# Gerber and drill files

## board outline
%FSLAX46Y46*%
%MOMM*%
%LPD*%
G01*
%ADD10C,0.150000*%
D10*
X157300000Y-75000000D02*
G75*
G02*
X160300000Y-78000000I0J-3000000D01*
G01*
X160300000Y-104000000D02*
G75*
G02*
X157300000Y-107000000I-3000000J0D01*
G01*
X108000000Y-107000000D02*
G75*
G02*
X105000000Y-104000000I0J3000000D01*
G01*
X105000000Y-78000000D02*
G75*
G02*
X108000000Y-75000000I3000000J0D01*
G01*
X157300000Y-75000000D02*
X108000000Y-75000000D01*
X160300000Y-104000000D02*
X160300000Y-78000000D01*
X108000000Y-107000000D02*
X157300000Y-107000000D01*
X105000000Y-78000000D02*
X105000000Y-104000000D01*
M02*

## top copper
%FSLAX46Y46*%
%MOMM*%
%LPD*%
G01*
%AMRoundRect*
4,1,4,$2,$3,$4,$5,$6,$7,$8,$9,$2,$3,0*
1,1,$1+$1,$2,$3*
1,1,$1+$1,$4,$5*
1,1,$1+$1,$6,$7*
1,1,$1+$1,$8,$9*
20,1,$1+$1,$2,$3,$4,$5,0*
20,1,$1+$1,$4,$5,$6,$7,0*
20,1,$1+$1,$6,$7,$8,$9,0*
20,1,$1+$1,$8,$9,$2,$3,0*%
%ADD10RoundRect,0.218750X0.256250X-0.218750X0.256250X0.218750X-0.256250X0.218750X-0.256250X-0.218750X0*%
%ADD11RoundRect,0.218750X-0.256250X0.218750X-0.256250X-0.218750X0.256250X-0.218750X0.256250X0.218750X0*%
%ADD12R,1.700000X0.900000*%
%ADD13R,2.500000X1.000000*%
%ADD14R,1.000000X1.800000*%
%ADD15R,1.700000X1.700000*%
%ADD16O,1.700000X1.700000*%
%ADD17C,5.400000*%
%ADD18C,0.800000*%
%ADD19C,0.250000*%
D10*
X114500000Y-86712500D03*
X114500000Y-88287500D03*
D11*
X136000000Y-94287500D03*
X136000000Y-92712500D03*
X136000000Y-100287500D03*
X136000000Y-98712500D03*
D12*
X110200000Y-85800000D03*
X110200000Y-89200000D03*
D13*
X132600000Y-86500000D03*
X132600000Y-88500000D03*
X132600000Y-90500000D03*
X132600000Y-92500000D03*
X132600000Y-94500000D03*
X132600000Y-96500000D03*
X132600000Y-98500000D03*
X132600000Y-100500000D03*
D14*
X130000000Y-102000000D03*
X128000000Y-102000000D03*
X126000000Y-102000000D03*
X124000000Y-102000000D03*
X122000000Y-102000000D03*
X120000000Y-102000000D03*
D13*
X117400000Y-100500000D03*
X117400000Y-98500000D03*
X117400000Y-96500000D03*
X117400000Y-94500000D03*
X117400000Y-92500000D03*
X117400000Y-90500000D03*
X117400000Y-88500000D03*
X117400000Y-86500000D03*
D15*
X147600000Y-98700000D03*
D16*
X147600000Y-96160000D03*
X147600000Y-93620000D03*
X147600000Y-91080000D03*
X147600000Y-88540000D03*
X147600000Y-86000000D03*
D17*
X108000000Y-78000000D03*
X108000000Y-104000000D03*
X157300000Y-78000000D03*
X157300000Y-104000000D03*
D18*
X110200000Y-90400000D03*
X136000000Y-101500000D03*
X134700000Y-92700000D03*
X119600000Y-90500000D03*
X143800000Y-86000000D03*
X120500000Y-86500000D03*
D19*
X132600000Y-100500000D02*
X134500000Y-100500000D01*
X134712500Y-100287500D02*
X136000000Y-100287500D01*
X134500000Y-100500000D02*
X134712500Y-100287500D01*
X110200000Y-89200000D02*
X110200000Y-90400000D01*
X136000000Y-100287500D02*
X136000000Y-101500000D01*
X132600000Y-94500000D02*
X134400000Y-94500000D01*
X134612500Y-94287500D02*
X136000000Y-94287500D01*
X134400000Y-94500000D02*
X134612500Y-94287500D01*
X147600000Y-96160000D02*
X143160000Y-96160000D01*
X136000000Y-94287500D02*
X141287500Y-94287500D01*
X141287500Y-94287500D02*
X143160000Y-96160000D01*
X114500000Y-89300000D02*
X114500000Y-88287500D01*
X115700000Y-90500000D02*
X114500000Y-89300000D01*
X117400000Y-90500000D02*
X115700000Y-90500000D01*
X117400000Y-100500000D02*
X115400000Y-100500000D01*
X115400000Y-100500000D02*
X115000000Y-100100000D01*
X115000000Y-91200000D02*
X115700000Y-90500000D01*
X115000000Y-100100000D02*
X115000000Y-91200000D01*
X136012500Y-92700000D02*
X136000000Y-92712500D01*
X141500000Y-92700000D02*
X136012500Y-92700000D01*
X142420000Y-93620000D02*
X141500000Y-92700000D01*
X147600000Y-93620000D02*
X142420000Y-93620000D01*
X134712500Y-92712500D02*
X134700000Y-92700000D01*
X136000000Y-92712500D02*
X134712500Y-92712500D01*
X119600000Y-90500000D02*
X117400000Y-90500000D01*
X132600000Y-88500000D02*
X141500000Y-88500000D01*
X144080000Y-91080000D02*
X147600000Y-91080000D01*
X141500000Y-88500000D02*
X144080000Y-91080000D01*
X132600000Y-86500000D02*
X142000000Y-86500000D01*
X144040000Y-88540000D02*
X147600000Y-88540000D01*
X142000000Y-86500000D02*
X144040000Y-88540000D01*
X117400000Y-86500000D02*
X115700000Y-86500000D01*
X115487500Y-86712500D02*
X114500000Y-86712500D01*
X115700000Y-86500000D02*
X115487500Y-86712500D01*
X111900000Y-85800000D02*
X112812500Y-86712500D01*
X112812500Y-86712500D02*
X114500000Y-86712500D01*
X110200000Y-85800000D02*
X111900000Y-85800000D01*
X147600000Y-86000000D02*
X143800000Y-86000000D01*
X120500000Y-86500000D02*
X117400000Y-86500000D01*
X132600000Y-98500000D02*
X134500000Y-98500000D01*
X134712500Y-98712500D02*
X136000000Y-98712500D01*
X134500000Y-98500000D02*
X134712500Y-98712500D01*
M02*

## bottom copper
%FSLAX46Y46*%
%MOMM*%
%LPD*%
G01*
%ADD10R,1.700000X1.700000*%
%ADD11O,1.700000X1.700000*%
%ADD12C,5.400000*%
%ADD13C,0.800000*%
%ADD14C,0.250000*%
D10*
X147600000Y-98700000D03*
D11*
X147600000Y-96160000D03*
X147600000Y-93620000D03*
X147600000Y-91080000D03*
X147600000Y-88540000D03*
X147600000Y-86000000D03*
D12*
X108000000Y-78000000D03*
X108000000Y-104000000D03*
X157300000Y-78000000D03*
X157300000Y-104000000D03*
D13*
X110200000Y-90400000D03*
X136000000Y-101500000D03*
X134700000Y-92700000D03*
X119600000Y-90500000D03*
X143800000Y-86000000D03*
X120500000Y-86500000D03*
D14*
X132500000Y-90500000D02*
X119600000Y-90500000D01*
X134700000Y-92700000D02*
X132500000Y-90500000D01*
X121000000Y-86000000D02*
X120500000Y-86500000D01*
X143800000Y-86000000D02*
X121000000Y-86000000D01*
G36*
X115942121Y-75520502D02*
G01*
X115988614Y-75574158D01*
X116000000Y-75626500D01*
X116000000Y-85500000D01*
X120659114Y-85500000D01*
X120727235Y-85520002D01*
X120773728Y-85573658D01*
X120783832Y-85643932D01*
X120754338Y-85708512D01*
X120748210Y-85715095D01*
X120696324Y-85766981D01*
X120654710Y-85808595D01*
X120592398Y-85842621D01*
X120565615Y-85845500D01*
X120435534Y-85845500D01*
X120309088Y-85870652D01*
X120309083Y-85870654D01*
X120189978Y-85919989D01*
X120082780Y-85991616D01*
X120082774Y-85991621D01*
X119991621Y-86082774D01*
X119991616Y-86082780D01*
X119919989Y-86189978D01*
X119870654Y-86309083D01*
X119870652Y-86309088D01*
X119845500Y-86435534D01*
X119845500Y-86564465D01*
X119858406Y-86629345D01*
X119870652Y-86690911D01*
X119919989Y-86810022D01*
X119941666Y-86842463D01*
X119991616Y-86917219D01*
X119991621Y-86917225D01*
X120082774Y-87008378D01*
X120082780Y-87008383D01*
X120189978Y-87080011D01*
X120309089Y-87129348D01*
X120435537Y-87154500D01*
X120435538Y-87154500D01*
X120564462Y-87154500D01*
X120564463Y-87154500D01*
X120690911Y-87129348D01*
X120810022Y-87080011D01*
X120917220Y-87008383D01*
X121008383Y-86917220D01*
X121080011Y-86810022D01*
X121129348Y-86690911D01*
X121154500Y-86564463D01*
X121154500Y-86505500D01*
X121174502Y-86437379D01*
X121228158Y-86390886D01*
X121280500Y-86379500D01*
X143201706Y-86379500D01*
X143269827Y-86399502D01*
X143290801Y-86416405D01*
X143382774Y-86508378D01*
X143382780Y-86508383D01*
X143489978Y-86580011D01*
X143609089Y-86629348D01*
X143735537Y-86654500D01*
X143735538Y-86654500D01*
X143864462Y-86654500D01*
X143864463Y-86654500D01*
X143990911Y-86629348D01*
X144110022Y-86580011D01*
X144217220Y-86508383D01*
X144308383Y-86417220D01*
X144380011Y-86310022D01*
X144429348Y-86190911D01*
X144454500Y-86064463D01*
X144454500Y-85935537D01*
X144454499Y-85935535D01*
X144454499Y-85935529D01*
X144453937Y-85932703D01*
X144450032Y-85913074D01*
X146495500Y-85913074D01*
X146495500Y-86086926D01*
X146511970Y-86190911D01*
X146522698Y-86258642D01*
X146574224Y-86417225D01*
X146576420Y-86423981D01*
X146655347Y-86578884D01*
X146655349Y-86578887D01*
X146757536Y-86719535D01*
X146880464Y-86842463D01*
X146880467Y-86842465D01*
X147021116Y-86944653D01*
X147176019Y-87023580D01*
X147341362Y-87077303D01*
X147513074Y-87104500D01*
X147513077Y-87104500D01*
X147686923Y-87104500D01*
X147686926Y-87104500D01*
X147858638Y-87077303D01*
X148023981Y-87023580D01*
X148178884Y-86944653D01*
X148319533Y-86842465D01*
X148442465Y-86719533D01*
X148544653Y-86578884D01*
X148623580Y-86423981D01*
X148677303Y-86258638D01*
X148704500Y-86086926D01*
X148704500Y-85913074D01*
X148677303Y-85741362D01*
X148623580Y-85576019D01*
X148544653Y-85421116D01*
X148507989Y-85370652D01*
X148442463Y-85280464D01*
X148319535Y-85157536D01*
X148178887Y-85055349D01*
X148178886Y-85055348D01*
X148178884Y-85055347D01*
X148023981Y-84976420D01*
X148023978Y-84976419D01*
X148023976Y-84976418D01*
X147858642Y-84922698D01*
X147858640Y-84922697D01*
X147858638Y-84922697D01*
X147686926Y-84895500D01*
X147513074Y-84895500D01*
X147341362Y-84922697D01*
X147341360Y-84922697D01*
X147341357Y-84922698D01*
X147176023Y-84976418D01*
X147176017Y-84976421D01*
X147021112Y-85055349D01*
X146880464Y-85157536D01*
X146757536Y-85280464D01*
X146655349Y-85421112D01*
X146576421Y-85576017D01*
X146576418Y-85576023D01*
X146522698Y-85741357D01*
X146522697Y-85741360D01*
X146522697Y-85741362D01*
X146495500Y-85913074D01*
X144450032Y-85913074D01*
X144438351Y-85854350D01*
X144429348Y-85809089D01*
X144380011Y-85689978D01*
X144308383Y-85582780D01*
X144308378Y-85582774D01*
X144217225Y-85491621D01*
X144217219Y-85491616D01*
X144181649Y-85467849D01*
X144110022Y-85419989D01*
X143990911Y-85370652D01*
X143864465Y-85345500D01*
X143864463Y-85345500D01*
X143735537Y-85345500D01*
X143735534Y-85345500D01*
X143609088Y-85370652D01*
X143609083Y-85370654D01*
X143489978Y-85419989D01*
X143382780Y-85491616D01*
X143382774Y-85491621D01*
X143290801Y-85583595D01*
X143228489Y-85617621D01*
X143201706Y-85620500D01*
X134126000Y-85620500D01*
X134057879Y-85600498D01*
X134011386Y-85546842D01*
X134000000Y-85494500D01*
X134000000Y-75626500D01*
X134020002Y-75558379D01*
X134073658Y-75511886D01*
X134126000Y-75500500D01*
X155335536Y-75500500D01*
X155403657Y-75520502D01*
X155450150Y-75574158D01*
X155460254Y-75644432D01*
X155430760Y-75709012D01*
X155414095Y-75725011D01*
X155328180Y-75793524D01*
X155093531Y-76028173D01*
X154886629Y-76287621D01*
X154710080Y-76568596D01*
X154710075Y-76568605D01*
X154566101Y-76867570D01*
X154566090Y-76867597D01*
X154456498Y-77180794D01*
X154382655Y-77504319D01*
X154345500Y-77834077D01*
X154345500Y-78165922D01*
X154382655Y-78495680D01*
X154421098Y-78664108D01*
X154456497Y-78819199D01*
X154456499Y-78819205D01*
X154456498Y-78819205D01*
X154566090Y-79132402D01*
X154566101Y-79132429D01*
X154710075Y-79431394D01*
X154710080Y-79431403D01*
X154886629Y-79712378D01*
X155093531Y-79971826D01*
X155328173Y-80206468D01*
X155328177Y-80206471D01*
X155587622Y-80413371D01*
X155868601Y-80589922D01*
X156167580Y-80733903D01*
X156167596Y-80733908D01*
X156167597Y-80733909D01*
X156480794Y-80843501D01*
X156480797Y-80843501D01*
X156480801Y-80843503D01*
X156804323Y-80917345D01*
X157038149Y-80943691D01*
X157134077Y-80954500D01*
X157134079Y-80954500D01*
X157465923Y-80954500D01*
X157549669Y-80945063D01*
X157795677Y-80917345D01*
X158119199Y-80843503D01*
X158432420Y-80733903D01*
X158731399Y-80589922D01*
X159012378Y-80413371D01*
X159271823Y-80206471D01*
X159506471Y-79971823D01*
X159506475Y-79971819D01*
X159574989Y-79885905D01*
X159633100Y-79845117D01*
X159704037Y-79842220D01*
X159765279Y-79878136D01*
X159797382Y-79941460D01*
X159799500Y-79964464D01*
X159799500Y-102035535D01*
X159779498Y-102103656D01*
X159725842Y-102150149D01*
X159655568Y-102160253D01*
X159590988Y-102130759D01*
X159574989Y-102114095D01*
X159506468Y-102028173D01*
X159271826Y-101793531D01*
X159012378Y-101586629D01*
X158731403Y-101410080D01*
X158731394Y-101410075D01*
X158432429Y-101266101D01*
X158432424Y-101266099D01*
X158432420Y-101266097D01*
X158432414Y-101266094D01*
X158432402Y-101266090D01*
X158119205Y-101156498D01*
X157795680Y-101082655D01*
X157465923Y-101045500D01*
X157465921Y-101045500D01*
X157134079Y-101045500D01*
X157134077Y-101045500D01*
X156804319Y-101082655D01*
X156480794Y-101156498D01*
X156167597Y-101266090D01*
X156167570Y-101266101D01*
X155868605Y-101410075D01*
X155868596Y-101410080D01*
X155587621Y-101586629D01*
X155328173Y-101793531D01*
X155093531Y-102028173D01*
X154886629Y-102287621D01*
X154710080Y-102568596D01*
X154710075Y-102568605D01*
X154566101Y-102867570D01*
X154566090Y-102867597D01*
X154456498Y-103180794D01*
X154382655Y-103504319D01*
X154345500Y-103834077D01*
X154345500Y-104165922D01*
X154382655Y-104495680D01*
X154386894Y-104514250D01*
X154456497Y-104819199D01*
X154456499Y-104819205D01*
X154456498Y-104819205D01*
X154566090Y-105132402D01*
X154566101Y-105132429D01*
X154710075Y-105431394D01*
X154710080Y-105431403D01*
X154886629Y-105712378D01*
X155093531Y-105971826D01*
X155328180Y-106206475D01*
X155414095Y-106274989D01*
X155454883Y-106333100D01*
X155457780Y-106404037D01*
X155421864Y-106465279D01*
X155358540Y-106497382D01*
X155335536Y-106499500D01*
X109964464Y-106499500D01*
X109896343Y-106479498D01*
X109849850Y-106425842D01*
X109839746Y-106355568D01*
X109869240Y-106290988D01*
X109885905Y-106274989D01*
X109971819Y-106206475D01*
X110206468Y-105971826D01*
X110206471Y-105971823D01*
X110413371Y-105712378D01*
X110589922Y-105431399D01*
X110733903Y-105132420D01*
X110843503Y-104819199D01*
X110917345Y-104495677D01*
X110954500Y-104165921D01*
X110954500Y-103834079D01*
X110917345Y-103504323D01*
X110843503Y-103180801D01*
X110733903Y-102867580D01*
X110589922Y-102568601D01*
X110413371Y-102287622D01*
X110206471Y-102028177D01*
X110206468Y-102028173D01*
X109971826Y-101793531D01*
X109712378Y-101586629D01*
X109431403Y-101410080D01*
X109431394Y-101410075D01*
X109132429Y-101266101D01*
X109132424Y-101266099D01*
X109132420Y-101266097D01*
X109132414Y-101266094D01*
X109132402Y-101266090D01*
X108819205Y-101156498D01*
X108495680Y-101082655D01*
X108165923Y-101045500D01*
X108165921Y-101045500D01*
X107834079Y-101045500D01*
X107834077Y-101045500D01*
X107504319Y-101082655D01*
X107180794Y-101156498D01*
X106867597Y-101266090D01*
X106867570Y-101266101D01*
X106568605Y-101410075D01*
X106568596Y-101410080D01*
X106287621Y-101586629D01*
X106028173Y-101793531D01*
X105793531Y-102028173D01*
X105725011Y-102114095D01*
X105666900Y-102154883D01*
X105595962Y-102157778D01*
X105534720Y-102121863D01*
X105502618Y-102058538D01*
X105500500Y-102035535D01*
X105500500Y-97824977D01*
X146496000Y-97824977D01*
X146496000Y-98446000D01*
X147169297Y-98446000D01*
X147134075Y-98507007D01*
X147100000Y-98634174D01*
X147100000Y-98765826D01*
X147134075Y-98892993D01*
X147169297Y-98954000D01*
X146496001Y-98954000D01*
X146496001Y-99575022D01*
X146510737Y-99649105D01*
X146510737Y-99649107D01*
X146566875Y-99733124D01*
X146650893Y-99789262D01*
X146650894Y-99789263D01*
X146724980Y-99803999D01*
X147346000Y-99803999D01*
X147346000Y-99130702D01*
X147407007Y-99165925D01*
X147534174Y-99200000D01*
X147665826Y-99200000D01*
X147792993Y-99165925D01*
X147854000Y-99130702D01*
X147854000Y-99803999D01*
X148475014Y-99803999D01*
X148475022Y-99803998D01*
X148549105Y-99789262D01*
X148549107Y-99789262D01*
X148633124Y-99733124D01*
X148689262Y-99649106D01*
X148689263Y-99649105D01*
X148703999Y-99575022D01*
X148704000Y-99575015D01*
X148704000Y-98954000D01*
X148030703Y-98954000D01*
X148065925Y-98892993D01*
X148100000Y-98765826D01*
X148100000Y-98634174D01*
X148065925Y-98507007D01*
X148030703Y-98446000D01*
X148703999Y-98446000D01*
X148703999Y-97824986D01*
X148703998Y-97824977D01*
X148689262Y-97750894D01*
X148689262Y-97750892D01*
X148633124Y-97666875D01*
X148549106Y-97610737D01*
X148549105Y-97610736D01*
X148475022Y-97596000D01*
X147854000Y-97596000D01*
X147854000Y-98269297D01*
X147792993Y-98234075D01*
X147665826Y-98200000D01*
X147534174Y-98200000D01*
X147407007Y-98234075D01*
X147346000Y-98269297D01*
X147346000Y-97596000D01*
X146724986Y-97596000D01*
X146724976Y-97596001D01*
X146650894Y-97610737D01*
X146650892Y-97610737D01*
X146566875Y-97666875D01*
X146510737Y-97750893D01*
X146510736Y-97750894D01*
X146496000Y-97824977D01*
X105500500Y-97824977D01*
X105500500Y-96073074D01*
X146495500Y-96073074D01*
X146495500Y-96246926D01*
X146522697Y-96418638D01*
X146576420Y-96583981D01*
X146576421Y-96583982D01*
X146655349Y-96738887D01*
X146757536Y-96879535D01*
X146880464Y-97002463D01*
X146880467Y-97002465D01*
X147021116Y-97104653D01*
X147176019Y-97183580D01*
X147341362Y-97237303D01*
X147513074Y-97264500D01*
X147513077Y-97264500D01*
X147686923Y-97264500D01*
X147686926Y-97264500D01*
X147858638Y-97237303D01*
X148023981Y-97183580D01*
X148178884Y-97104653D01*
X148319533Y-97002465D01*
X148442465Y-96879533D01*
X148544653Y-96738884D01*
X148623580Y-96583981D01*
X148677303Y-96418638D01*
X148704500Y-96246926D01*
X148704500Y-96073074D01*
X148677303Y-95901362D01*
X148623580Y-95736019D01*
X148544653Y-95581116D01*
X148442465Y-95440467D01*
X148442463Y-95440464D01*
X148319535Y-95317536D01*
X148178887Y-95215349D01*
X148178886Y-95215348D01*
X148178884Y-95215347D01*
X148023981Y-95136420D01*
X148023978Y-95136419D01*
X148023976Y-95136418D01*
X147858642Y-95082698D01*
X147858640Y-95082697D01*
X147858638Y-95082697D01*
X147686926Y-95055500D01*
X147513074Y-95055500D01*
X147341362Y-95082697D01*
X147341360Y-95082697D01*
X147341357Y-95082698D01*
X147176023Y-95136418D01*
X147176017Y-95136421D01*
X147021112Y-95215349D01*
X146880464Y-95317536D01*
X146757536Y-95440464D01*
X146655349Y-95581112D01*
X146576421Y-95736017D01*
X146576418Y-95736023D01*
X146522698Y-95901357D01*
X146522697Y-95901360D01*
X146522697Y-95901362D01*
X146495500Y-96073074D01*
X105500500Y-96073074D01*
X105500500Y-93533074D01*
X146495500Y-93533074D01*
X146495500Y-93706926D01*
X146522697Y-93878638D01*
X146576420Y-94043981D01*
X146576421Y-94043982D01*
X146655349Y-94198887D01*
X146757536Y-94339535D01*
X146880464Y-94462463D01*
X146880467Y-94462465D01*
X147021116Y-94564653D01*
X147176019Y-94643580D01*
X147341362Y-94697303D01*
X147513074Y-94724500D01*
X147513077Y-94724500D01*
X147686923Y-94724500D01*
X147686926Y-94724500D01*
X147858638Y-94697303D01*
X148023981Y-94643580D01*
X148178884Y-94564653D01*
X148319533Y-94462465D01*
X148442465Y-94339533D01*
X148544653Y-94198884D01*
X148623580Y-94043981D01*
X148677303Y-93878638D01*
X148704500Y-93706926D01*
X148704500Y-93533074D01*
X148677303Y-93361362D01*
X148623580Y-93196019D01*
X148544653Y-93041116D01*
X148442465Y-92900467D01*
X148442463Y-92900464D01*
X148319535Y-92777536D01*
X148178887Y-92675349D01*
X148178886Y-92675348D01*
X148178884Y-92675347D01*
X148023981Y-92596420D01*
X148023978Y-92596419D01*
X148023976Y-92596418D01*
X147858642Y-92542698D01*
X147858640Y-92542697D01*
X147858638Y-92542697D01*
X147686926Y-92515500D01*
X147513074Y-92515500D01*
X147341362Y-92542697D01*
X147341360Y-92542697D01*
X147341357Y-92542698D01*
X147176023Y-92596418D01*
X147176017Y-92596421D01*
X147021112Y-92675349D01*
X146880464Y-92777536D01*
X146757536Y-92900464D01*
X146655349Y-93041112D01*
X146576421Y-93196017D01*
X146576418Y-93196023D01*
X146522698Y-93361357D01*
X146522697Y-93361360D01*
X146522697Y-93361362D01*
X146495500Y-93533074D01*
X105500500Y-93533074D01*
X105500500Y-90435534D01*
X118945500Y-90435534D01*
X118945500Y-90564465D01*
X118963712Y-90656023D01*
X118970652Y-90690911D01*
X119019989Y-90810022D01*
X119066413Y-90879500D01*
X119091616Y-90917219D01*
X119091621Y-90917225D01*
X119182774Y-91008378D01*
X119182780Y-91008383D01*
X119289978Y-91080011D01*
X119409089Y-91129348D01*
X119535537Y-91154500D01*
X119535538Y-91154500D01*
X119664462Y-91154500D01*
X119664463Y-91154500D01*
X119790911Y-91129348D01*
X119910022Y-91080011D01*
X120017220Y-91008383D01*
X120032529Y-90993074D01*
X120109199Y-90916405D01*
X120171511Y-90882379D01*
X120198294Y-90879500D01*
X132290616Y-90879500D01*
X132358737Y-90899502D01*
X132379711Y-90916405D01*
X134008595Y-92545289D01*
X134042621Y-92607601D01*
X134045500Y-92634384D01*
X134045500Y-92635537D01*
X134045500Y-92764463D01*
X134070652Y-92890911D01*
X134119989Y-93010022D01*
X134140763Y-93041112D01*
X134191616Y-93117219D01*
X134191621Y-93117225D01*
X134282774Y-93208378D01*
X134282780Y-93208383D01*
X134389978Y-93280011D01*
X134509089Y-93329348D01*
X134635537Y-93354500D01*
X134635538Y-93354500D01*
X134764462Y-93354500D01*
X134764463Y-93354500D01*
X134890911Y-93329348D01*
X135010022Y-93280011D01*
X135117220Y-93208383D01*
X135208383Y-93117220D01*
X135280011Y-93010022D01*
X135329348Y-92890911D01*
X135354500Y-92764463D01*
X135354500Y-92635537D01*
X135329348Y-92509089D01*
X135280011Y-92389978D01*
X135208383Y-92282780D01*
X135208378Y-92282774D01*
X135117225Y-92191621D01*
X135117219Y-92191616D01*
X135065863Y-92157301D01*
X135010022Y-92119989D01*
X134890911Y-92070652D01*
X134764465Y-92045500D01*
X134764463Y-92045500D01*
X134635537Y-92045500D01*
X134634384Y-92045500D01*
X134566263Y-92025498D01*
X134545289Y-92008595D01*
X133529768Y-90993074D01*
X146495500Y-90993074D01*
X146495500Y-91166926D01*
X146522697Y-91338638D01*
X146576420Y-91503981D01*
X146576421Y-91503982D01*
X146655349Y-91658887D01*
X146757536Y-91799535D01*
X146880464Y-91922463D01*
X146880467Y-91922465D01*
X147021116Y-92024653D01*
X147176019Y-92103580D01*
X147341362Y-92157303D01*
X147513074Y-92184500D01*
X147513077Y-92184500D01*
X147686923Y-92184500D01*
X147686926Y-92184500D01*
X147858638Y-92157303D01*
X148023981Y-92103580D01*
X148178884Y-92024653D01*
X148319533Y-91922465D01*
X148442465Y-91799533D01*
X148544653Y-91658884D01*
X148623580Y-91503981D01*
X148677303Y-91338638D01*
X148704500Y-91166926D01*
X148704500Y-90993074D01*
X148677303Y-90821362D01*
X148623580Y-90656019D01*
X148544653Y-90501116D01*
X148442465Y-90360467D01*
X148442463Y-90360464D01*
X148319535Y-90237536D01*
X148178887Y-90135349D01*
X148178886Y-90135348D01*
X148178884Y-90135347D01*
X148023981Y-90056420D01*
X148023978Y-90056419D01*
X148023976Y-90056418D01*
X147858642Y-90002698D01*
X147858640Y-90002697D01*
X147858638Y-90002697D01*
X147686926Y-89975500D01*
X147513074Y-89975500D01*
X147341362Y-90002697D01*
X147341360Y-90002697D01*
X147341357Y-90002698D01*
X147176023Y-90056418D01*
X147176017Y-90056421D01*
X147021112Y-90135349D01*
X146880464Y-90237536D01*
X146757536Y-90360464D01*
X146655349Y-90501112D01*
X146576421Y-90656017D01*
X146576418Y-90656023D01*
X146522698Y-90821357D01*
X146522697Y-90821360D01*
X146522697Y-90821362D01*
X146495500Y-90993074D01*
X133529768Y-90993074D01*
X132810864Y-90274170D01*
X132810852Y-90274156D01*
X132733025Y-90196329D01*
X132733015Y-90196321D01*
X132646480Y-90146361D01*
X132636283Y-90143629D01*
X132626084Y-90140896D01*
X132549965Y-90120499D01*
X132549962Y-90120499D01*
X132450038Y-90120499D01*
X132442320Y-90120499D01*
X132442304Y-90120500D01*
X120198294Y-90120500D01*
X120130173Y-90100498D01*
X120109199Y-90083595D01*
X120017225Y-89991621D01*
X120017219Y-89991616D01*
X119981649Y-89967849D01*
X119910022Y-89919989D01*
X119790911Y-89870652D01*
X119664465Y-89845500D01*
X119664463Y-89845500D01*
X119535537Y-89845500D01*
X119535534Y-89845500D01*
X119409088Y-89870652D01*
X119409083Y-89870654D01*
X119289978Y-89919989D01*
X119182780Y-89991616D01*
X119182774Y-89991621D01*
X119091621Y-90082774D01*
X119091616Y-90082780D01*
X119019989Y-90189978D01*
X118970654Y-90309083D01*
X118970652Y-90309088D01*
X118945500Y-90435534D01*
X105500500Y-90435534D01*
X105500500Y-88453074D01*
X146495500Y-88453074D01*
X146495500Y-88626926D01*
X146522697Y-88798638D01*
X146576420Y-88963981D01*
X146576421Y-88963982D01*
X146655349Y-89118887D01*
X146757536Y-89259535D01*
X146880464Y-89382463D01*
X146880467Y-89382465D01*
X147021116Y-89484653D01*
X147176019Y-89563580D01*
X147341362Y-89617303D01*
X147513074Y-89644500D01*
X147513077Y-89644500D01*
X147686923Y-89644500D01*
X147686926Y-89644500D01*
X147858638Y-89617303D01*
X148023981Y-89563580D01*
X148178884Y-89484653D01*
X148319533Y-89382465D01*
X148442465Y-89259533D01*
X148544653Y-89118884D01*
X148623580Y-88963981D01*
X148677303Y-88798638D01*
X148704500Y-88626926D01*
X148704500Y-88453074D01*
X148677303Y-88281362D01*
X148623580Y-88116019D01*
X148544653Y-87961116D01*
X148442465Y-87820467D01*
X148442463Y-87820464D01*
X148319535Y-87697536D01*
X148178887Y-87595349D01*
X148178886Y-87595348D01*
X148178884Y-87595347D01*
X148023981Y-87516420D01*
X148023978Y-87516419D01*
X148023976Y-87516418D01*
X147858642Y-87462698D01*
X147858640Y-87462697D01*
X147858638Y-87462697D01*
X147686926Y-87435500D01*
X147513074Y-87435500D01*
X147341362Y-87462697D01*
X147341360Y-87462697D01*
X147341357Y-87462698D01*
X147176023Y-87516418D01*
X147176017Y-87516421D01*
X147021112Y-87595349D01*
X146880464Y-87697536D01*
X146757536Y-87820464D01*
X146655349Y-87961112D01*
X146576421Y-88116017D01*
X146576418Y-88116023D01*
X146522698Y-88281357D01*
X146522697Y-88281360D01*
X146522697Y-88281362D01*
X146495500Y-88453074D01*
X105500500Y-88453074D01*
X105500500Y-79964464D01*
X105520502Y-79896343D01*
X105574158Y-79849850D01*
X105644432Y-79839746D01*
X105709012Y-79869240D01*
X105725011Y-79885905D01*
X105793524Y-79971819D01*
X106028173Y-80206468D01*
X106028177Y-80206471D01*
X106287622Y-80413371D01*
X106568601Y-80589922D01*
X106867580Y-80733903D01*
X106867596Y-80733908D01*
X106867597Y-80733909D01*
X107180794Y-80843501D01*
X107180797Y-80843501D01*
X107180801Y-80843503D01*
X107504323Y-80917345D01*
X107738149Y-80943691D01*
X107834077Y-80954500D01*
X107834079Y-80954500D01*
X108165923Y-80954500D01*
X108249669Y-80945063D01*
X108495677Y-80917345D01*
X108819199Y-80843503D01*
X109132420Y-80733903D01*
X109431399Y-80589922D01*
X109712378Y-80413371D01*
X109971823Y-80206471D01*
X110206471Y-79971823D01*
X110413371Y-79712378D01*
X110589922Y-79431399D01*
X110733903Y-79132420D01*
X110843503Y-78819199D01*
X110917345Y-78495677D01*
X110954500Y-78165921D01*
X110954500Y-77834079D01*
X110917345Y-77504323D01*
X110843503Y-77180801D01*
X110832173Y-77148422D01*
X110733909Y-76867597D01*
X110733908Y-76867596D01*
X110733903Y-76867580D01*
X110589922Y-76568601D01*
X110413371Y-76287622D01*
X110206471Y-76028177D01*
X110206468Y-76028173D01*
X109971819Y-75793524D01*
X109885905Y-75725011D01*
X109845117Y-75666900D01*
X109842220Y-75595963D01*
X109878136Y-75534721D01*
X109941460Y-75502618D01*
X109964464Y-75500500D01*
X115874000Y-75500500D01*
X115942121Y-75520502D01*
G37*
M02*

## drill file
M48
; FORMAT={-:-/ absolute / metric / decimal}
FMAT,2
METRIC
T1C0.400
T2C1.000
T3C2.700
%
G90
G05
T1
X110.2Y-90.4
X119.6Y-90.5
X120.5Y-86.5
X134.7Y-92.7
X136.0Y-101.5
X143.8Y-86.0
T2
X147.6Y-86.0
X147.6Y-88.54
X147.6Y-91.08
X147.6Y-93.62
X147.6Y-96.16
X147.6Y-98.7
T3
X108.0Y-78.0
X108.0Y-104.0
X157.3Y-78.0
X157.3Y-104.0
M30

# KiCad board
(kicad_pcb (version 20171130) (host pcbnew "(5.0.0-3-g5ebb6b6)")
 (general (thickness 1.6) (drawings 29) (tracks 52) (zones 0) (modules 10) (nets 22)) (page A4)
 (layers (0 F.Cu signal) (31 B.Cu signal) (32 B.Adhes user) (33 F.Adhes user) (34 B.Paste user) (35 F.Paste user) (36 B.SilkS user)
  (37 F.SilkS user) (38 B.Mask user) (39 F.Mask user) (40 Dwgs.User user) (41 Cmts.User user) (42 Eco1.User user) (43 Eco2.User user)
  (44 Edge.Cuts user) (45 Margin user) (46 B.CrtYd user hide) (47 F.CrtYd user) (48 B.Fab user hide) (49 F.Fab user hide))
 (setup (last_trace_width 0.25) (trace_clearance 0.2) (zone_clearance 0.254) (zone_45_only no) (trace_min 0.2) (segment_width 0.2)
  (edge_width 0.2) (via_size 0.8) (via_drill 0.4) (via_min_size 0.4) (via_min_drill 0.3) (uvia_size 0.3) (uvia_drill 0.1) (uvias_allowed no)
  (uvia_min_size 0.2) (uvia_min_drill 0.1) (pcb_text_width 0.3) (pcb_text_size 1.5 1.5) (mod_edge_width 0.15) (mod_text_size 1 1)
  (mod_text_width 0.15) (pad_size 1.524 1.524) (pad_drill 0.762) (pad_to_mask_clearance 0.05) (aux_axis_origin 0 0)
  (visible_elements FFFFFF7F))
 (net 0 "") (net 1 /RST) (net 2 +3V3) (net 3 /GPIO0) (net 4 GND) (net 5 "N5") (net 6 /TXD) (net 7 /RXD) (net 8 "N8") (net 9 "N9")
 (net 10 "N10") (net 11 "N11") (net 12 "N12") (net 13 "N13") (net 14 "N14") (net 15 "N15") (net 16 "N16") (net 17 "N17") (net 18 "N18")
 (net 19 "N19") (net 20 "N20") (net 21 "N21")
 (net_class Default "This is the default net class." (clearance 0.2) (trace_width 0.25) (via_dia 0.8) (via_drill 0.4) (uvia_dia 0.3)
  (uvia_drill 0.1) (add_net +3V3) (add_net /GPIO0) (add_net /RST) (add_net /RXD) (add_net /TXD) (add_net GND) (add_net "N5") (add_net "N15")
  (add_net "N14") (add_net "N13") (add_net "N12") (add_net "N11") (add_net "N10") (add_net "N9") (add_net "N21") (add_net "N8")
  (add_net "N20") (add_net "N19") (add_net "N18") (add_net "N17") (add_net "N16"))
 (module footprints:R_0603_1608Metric (layer F.Cu) (at 114.5 87.5 90)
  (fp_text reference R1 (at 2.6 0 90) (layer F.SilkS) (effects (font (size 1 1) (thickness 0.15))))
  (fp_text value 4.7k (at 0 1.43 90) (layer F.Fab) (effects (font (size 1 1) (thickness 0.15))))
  (pad 2 smd roundrect (at 0.7875 0 90) (size 0.875 0.95) (layers F.Cu F.Paste F.Mask) (roundrect_rratio 0.25) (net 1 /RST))
  (pad 1 smd roundrect (at -0.7875 0 90) (size 0.875 0.95) (layers F.Cu F.Paste F.Mask) (roundrect_rratio 0.25) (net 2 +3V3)))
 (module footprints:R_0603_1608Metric (layer F.Cu) (at 136 93.5 270)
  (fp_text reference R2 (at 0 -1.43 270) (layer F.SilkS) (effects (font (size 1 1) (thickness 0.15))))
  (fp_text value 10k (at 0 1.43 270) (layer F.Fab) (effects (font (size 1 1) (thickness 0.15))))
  (pad 2 smd roundrect (at 0.7875 0 270) (size 0.875 0.95) (layers F.Cu F.Paste F.Mask) (roundrect_rratio 0.25) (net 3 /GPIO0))
  (pad 1 smd roundrect (at -0.7875 0 270) (size 0.875 0.95) (layers F.Cu F.Paste F.Mask) (roundrect_rratio 0.25) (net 2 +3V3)))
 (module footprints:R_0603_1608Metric (layer F.Cu) (at 136 99.5 270)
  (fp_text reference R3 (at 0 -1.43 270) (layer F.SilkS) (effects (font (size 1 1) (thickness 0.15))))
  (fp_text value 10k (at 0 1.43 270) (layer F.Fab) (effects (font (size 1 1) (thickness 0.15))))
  (pad 2 smd roundrect (at 0.7875 0 270) (size 0.875 0.95) (layers F.Cu F.Paste F.Mask) (roundrect_rratio 0.25) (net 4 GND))
  (pad 1 smd roundrect (at -0.7875 0 270) (size 0.875 0.95) (layers F.Cu F.Paste F.Mask) (roundrect_rratio 0.25) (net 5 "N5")))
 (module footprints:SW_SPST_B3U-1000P (layer F.Cu) (at 110.2 87.5 90)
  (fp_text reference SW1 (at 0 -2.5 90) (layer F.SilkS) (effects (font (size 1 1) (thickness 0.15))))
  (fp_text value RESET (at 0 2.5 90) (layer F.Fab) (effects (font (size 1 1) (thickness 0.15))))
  (pad 2 smd rect (at 1.7 0 90) (size 0.9 1.7) (layers F.Cu F.Paste F.Mask) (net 1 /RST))
  (pad 1 smd rect (at -1.7 0 90) (size 0.9 1.7) (layers F.Cu F.Paste F.Mask) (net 4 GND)))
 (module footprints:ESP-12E (layer F.Cu) (at 125 90)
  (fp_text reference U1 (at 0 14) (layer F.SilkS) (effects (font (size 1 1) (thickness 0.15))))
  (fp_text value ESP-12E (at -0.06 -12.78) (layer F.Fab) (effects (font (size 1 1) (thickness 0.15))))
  (pad 22 smd rect (at 7.6 -3.5) (size 2.5 1) (layers F.Cu F.Paste F.Mask) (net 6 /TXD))
  (pad 21 smd rect (at 7.6 -1.5) (size 2.5 1) (layers F.Cu F.Paste F.Mask) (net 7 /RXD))
  (pad 20 smd rect (at 7.6 0.5) (size 2.5 1) (layers F.Cu F.Paste F.Mask) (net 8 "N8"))
  (pad 19 smd rect (at 7.6 2.5) (size 2.5 1) (layers F.Cu F.Paste F.Mask) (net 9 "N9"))
  (pad 18 smd rect (at 7.6 4.5) (size 2.5 1) (layers F.Cu F.Paste F.Mask) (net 3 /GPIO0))
  (pad 17 smd rect (at 7.6 6.5) (size 2.5 1) (layers F.Cu F.Paste F.Mask) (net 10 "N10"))
  (pad 16 smd rect (at 7.6 8.5) (size 2.5 1) (layers F.Cu F.Paste F.Mask) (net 5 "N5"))
  (pad 15 smd rect (at 7.6 10.5) (size 2.5 1) (layers F.Cu F.Paste F.Mask) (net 4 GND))
  (pad 14 smd rect (at 5 12) (size 1 1.8) (layers F.Cu F.Paste F.Mask) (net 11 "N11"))
  (pad 13 smd rect (at 3 12) (size 1 1.8) (layers F.Cu F.Paste F.Mask) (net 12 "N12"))
  (pad 12 smd rect (at 1 12) (size 1 1.8) (layers F.Cu F.Paste F.Mask) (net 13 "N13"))
  (pad 11 smd rect (at -1 12) (size 1 1.8) (layers F.Cu F.Paste F.Mask) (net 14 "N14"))
  (pad 10 smd rect (at -3 12) (size 1 1.8) (layers F.Cu F.Paste F.Mask) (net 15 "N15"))
  (pad 9 smd rect (at -5 12) (size 1 1.8) (layers F.Cu F.Paste F.Mask) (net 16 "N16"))
  (pad 8 smd rect (at -7.6 10.5) (size 2.5 1) (layers F.Cu F.Paste F.Mask) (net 2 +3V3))
  (pad 7 smd rect (at -7.6 8.5) (size 2.5 1) (layers F.Cu F.Paste F.Mask) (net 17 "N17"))
  (pad 6 smd rect (at -7.6 6.5) (size 2.5 1) (layers F.Cu F.Paste F.Mask) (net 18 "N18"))
  (pad 5 smd rect (at -7.6 4.5) (size 2.5 1) (layers F.Cu F.Paste F.Mask) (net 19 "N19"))
  (pad 4 smd rect (at -7.6 2.5) (size 2.5 1) (layers F.Cu F.Paste F.Mask) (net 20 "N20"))
  (pad 3 smd rect (at -7.6 0.5) (size 2.5 1) (layers F.Cu F.Paste F.Mask) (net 2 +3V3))
  (pad 2 smd rect (at -7.6 -1.5) (size 2.5 1) (layers F.Cu F.Paste F.Mask) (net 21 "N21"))
  (pad 1 smd rect (at -7.6 -3.5) (size 2.5 1) (layers F.Cu F.Paste F.Mask) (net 1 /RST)))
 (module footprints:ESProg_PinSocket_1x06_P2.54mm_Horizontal (layer F.Cu) (at 147.6 98.7)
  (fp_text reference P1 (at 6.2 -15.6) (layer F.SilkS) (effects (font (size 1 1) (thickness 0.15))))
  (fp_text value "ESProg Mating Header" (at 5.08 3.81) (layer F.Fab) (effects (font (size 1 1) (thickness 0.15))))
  (pad 1 thru_hole rect (at 0 0 180) (size 1.7 1.7) (drill 1) (layers *.Cu *.Mask) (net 4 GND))
  (pad 2 thru_hole oval (at 0 -2.54 180) (size 1.7 1.7) (drill 1) (layers *.Cu *.Mask) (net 3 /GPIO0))
  (pad 3 thru_hole oval (at 0 -5.08 180) (size 1.7 1.7) (drill 1) (layers *.Cu *.Mask) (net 2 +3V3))
  (pad 4 thru_hole oval (at 0 -7.62 180) (size 1.7 1.7) (drill 1) (layers *.Cu *.Mask) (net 7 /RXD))
  (pad 5 thru_hole oval (at 0 -10.16 180) (size 1.7 1.7) (drill 1) (layers *.Cu *.Mask) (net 6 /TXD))
  (pad 6 thru_hole oval (at 0 -12.7 180) (size 1.7 1.7) (drill 1) (layers *.Cu *.Mask) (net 1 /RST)))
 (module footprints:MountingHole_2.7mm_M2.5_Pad (layer F.Cu) (at 108 78)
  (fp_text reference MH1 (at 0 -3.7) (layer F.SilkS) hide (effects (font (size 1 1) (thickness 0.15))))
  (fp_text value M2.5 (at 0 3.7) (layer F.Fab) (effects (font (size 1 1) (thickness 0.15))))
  (pad 1 thru_hole circle (at 0 0) (size 5.4 5.4) (drill 2.7) (layers *.Cu *.Mask)))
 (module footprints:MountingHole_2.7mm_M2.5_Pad (layer F.Cu) (at 108 104)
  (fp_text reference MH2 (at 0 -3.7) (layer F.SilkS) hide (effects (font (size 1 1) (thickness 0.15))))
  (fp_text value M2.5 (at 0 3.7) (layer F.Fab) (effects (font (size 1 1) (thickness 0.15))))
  (pad 1 thru_hole circle (at 0 0) (size 5.4 5.4) (drill 2.7) (layers *.Cu *.Mask)))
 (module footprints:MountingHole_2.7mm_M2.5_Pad (layer F.Cu) (at 157.3 78)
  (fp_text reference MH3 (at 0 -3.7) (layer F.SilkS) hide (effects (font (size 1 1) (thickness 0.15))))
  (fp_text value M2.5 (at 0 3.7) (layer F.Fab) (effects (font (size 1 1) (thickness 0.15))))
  (pad 1 thru_hole circle (at 0 0) (size 5.4 5.4) (drill 2.7) (layers *.Cu *.Mask)))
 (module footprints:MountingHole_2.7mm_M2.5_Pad (layer F.Cu) (at 157.3 104)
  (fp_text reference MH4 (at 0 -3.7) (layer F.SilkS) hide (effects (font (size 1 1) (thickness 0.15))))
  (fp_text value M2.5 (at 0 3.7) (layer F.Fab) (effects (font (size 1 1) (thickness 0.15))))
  (pad 1 thru_hole circle (at 0 0) (size 5.4 5.4) (drill 2.7) (layers *.Cu *.Mask)))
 (gr_arc (start 157.3 78) (end 160.3 78) (angle -90) (layer Edge.Cuts) (width 0.15))
 (gr_arc (start 157.3 104) (end 157.3 107) (angle -90) (layer Edge.Cuts) (width 0.15))
 (gr_arc (start 108 104) (end 105 104) (angle -90) (layer Edge.Cuts) (width 0.15))
 (gr_arc (start 108 78) (end 108 75) (angle -90) (layer Edge.Cuts) (width 0.15))
 (gr_line (start 157.3 75) (end 108 75) (layer Edge.Cuts) (width 0.15))
 (gr_line (start 160.3 104) (end 160.3 78) (layer Edge.Cuts) (width 0.15))
 (gr_line (start 108 107) (end 157.3 107) (layer Edge.Cuts) (width 0.15))
 (gr_line (start 105 78) (end 105 104) (layer Edge.Cuts) (width 0.15))
 (segment (start 132.6 100.5) (end 134.5 100.5) (width 0.25) (layer F.Cu) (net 4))
 (segment (start 134.7125 100.2875) (end 136 100.2875) (width 0.25) (layer F.Cu) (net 4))
 (segment (start 134.5 100.5) (end 134.7125 100.2875) (width 0.25) (layer F.Cu) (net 4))
 (via (at 110.2 90.4) (size 0.8) (drill 0.4) (layers F.Cu B.Cu) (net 4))
 (segment (start 110.2 89.2) (end 110.2 90.4) (width 0.25) (layer F.Cu) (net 4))
 (via (at 136 101.5) (size 0.8) (drill 0.4) (layers F.Cu B.Cu) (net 4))
 (segment (start 136 100.2875) (end 136 101.5) (width 0.25) (layer F.Cu) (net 4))
 (segment (start 132.6 94.5) (end 134.4 94.5) (width 0.25) (layer F.Cu) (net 3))
 (segment (start 134.6125 94.2875) (end 136 94.2875) (width 0.25) (layer F.Cu) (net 3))
 (segment (start 134.4 94.5) (end 134.6125 94.2875) (width 0.25) (layer F.Cu) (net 3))
 (segment (start 147.6 96.16) (end 143.16 96.16) (width 0.25) (layer F.Cu) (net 3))
 (segment (start 136 94.2875) (end 141.2875 94.2875) (width 0.25) (layer F.Cu) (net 3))
 (segment (start 141.2875 94.2875) (end 143.16 96.16) (width 0.25) (layer F.Cu) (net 3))
 (segment (start 114.5 89.3) (end 114.5 88.2875) (width 0.25) (layer F.Cu) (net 2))
 (segment (start 115.7 90.5) (end 114.5 89.3) (width 0.25) (layer F.Cu) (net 2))
 (segment (start 117.4 90.5) (end 115.7 90.5) (width 0.25) (layer F.Cu) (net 2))
 (segment (start 117.4 100.5) (end 115.4 100.5) (width 0.25) (layer F.Cu) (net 2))
 (segment (start 115.4 100.5) (end 115 100.1) (width 0.25) (layer F.Cu) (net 2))
 (segment (start 115 91.2) (end 115.7 90.5) (width 0.25) (layer F.Cu) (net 2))
 (segment (start 115 100.1) (end 115 91.2) (width 0.25) (layer F.Cu) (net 2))
 (segment (start 136.0125 92.7) (end 136 92.7125) (width 0.25) (layer F.Cu) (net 2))
 (segment (start 141.5 92.7) (end 136.0125 92.7) (width 0.25) (layer F.Cu) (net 2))
 (segment (start 142.42 93.62) (end 141.5 92.7) (width 0.25) (layer F.Cu) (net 2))
 (segment (start 147.6 93.62) (end 142.42 93.62) (width 0.25) (layer F.Cu) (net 2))
 (via (at 134.7 92.7) (size 0.8) (drill 0.4) (layers F.Cu B.Cu) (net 2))
 (segment (start 134.7125 92.7125) (end 134.7 92.7) (width 0.25) (layer F.Cu) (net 2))
 (segment (start 136 92.7125) (end 134.7125 92.7125) (width 0.25) (layer F.Cu) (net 2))
 (via (at 119.6 90.5) (size 0.8) (drill 0.4) (layers F.Cu B.Cu) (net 2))
 (segment (start 132.5 90.5) (end 119.6 90.5) (width 0.25) (layer B.Cu) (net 2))
 (segment (start 134.7 92.7) (end 132.5 90.5) (width 0.25) (layer B.Cu) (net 2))
 (segment (start 119.6 90.5) (end 117.4 90.5) (width 0.25) (layer F.Cu) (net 2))
 (segment (start 132.6 88.5) (end 141.5 88.5) (width 0.25) (layer F.Cu) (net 7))
 (segment (start 144.08 91.08) (end 147.6 91.08) (width 0.25) (layer F.Cu) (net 7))
 (segment (start 141.5 88.5) (end 144.08 91.08) (width 0.25) (layer F.Cu) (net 7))
 (segment (start 132.6 86.5) (end 142 86.5) (width 0.25) (layer F.Cu) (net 6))
 (segment (start 144.04 88.54) (end 147.6 88.54) (width 0.25) (layer F.Cu) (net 6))
 (segment (start 142 86.5) (end 144.04 88.54) (width 0.25) (layer F.Cu) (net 6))
 (segment (start 117.4 86.5) (end 115.7 86.5) (width 0.25) (layer F.Cu) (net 1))
 (segment (start 115.4875 86.7125) (end 114.5 86.7125) (width 0.25) (layer F.Cu) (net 1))
 (segment (start 115.7 86.5) (end 115.4875 86.7125) (width 0.25) (layer F.Cu) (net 1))
 (segment (start 111.9 85.8) (end 112.8125 86.7125) (width 0.25) (layer F.Cu) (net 1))
 (segment (start 112.8125 86.7125) (end 114.5 86.7125) (width 0.25) (layer F.Cu) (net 1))
 (segment (start 110.2 85.8) (end 111.9 85.8) (width 0.25) (layer F.Cu) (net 1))
 (via (at 143.8 86) (size 0.8) (drill 0.4) (layers F.Cu B.Cu) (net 1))
 (segment (start 147.6 86) (end 143.8 86) (width 0.25) (layer F.Cu) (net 1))
 (segment (start 121 86) (end 120.5 86.5) (width 0.25) (layer B.Cu) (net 1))
 (via (at 120.5 86.5) (size 0.8) (drill 0.4) (layers F.Cu B.Cu) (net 1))
 (segment (start 143.8 86) (end 121 86) (width 0.25) (layer B.Cu) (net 1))
 (segment (start 120.5 86.5) (end 117.4 86.5) (width 0.25) (layer F.Cu) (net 1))
 (segment (start 132.6 98.5) (end 134.5 98.5) (width 0.25) (layer F.Cu) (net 5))
 (segment (start 134.7125 98.7125) (end 136 98.7125) (width 0.25) (layer F.Cu) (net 5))
 (segment (start 134.5 98.5) (end 134.7125 98.7125) (width 0.25) (layer F.Cu) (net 5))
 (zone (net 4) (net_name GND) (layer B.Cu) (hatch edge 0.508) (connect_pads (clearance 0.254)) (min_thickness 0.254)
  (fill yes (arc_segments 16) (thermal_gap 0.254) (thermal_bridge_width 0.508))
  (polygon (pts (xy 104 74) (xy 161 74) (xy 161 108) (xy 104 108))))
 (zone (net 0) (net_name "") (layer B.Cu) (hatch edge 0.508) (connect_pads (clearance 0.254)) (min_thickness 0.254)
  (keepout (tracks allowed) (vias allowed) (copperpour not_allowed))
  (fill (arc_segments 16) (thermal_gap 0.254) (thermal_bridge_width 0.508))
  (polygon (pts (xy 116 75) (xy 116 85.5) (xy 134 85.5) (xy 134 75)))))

